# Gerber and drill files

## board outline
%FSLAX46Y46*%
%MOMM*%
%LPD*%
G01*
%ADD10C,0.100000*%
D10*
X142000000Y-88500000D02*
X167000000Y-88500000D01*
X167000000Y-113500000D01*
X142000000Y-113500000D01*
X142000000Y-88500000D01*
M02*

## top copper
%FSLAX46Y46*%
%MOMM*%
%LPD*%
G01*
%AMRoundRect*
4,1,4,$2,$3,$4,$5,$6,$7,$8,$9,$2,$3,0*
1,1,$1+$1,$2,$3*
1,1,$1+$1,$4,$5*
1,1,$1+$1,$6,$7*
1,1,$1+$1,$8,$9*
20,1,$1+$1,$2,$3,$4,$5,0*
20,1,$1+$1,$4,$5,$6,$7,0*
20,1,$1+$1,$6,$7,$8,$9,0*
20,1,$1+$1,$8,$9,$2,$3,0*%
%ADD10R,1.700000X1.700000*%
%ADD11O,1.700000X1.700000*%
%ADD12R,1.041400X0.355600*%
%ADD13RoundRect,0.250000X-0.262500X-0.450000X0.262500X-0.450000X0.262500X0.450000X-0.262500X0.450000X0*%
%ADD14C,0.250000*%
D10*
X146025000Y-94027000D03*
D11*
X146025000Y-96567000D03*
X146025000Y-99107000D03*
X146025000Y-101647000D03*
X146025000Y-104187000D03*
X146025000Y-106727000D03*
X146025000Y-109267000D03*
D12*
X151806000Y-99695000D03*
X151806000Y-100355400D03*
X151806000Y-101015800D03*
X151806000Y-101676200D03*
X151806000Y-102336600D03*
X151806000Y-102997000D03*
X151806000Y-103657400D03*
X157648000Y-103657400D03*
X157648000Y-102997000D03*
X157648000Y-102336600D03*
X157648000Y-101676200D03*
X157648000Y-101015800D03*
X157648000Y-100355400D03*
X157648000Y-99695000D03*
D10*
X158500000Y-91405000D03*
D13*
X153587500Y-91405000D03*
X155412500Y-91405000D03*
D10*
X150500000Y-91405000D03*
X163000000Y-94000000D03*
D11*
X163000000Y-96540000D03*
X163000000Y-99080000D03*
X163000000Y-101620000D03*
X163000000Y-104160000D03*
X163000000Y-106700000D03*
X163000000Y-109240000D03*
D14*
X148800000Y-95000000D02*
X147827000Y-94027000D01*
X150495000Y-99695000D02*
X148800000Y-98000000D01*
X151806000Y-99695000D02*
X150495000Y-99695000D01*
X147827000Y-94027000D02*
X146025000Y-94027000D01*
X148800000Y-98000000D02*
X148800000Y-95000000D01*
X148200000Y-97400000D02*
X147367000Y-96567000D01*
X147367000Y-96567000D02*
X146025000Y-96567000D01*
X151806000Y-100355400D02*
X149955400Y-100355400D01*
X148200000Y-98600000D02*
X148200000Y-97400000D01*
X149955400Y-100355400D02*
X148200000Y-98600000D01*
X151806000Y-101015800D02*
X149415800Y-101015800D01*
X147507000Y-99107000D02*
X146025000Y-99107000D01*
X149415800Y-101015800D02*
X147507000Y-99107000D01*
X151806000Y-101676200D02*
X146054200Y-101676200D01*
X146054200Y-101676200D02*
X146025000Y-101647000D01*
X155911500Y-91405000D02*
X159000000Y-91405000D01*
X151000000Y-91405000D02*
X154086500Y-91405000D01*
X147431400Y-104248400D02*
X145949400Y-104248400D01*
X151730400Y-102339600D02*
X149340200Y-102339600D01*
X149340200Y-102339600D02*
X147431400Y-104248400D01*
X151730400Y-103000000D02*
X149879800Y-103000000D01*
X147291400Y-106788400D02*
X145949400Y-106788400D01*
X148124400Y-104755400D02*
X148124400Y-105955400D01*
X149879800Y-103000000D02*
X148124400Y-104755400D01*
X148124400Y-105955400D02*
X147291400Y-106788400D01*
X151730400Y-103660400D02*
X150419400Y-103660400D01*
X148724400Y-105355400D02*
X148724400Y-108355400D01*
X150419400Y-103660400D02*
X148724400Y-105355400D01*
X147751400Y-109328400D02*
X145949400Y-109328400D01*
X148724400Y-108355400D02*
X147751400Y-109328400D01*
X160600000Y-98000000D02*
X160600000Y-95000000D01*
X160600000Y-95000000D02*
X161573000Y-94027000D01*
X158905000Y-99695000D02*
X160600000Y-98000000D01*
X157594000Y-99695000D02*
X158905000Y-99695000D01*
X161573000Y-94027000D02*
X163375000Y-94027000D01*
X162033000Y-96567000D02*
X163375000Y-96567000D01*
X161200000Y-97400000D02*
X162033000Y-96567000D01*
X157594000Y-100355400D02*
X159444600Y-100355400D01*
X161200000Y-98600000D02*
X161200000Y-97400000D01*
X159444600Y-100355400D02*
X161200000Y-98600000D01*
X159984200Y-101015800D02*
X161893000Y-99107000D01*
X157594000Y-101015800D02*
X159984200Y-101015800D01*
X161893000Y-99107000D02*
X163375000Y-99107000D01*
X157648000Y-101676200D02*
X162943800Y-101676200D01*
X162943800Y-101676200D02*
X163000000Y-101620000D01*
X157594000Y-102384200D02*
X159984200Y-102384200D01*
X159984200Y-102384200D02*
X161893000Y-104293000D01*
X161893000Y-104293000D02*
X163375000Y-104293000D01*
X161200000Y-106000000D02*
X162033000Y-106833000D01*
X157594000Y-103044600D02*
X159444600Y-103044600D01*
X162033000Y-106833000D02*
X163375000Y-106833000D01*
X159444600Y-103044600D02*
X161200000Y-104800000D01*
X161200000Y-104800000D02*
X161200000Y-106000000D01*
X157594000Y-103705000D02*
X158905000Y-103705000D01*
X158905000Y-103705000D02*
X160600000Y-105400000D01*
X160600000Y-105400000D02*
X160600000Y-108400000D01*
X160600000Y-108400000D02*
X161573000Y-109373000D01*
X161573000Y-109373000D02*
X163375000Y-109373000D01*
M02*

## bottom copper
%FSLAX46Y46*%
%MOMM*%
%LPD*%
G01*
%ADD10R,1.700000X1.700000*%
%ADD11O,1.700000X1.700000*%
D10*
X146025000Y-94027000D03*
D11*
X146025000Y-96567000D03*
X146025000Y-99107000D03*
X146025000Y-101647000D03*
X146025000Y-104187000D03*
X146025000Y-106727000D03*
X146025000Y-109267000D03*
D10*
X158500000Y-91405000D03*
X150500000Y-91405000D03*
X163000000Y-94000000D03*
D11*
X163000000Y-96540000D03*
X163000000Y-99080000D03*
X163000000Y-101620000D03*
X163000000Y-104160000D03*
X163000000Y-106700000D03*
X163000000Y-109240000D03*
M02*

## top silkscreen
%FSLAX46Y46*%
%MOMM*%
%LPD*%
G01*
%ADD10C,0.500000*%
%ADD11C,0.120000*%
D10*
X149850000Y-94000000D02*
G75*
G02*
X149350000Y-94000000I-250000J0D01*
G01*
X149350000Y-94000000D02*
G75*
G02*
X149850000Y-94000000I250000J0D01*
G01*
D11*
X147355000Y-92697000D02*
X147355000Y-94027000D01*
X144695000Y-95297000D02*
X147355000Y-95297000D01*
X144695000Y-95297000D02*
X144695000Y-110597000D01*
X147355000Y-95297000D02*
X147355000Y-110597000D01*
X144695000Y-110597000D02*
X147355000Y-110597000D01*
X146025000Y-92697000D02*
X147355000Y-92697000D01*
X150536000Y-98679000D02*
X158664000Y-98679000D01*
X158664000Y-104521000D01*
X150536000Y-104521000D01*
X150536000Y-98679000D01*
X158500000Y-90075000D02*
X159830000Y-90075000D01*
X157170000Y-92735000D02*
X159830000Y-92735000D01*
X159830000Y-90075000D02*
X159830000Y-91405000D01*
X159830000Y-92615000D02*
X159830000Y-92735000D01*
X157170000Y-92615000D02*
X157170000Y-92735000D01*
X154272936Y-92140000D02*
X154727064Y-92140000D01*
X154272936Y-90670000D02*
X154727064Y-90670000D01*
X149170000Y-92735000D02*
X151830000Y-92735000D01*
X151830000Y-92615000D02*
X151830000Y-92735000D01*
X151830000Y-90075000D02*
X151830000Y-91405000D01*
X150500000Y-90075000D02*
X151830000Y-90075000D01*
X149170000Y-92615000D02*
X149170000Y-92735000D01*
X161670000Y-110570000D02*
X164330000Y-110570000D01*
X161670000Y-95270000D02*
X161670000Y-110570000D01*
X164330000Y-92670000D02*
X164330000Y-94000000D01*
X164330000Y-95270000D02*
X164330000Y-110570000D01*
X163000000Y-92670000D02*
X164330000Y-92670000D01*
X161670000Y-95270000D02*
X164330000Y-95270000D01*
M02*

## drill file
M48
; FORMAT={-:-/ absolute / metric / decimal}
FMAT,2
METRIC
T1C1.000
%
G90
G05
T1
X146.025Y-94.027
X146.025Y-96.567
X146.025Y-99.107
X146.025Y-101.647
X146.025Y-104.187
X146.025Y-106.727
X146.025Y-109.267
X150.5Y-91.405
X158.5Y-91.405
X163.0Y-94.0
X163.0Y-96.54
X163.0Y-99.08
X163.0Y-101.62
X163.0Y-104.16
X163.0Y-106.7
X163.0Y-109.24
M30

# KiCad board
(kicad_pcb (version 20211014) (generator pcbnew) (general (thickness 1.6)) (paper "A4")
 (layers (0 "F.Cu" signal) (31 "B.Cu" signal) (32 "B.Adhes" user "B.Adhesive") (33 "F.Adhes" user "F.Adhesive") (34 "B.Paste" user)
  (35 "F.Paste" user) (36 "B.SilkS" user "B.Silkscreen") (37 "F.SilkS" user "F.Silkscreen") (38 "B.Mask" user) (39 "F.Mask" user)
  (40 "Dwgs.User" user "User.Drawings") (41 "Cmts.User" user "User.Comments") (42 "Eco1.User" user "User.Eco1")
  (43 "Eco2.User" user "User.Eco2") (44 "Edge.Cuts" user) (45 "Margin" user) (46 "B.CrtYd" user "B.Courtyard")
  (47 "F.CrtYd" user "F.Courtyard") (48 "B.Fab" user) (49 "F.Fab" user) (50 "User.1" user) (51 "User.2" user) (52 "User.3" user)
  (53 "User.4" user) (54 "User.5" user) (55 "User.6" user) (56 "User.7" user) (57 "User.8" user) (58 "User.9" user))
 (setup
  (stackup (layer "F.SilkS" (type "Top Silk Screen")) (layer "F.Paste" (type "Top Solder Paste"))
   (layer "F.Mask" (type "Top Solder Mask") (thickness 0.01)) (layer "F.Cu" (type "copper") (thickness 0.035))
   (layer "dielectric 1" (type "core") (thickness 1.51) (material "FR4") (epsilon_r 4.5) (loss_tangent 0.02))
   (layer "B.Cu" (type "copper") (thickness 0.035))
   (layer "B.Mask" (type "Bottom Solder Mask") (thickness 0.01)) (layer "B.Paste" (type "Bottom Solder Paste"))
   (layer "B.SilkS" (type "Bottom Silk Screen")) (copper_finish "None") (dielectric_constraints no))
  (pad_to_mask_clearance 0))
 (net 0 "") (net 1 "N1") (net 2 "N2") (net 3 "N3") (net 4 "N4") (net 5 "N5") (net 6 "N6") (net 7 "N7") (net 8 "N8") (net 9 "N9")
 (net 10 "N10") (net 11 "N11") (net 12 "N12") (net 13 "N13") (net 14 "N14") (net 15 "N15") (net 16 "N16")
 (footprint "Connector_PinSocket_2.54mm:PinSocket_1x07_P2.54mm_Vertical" (layer "F.Cu") (at 146.025 94.027)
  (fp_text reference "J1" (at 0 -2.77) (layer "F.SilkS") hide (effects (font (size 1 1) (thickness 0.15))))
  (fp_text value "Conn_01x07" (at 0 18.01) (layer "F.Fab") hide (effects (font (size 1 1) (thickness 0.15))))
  (fp_line (start 1.33 -1.33) (end 1.33 0) (layer "F.SilkS") (width 0.12))
  (fp_line (start -1.33 1.27) (end 1.33 1.27) (layer "F.SilkS") (width 0.12))
  (fp_line (start -1.33 1.27) (end -1.33 16.57) (layer "F.SilkS") (width 0.12))
  (fp_line (start 1.33 1.27) (end 1.33 16.57) (layer "F.SilkS") (width 0.12))
  (fp_line (start -1.33 16.57) (end 1.33 16.57) (layer "F.SilkS") (width 0.12))
  (fp_line (start 0 -1.33) (end 1.33 -1.33) (layer "F.SilkS") (width 0.12))
  (pad "1" thru_hole rect (at 0 0) (size 1.7 1.7) (drill 1) (layers *.Cu *.Mask) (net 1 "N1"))
  (pad "2" thru_hole oval (at 0 2.54) (size 1.7 1.7) (drill 1) (layers *.Cu *.Mask) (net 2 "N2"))
  (pad "3" thru_hole oval (at 0 5.08) (size 1.7 1.7) (drill 1) (layers *.Cu *.Mask) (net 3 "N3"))
  (pad "4" thru_hole oval (at 0 7.62) (size 1.7 1.7) (drill 1) (layers *.Cu *.Mask) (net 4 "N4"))
  (pad "5" thru_hole oval (at 0 10.16) (size 1.7 1.7) (drill 1) (layers *.Cu *.Mask) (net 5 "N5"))
  (pad "6" thru_hole oval (at 0 12.7) (size 1.7 1.7) (drill 1) (layers *.Cu *.Mask) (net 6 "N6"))
  (pad "7" thru_hole oval (at 0 15.24) (size 1.7 1.7) (drill 1) (layers *.Cu *.Mask) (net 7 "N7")))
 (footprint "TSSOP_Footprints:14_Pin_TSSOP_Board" (layer "F.Cu") (at 154.727 103.759)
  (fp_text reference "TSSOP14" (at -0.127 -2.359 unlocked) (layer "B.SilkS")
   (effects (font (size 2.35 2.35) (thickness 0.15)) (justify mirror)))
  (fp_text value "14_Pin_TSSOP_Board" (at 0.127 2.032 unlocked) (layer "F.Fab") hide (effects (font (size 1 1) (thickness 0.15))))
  (fp_rect (start -4.191 -5.08) (end 3.937 0.762) (layer "F.SilkS") (width 0.12) (fill none))
  (pad "1" smd rect (at -2.921 -4.064) (size 1.0414 0.3556) (layers "F.Cu" "F.Paste" "F.Mask") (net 1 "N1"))
  (pad "2" smd rect (at -2.921 -3.4036) (size 1.0414 0.3556) (layers "F.Cu" "F.Paste" "F.Mask") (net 2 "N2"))
  (pad "3" smd rect (at -2.921 -2.7432) (size 1.0414 0.3556) (layers "F.Cu" "F.Paste" "F.Mask") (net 3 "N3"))
  (pad "4" smd rect (at -2.921 -2.0828) (size 1.0414 0.3556) (layers "F.Cu" "F.Paste" "F.Mask") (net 4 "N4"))
  (pad "5" smd rect (at -2.921 -1.4224) (size 1.0414 0.3556) (layers "F.Cu" "F.Paste" "F.Mask") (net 5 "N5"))
  (pad "6" smd rect (at -2.921 -0.762) (size 1.0414 0.3556) (layers "F.Cu" "F.Paste" "F.Mask") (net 6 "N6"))
  (pad "7" smd rect (at -2.921 -0.1016) (size 1.0414 0.3556) (layers "F.Cu" "F.Paste" "F.Mask") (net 7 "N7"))
  (pad "8" smd rect (at 2.921 -0.1016) (size 1.0414 0.3556) (layers "F.Cu" "F.Paste" "F.Mask") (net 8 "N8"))
  (pad "9" smd rect (at 2.921 -0.762) (size 1.0414 0.3556) (layers "F.Cu" "F.Paste" "F.Mask") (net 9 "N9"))
  (pad "10" smd rect (at 2.921 -1.4224) (size 1.0414 0.3556) (layers "F.Cu" "F.Paste" "F.Mask") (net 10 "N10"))
  (pad "11" smd rect (at 2.921 -2.0828) (size 1.0414 0.3556) (layers "F.Cu" "F.Paste" "F.Mask") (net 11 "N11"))
  (pad "12" smd rect (at 2.921 -2.7432) (size 1.0414 0.3556) (layers "F.Cu" "F.Paste" "F.Mask") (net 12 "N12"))
  (pad "13" smd rect (at 2.921 -3.4036) (size 1.0414 0.3556) (layers "F.Cu" "F.Paste" "F.Mask") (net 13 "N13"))
  (pad "14" smd rect (at 2.921 -4.064) (size 1.0414 0.3556) (layers "F.Cu" "F.Paste" "F.Mask") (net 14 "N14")))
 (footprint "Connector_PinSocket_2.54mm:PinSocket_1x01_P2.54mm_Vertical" (layer "F.Cu") (at 158.5 91.405)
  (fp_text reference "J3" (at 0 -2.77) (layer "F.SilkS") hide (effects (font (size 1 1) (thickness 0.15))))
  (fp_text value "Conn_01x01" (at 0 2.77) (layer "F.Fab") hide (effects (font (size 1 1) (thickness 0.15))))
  (fp_line (start 0 -1.33) (end 1.33 -1.33) (layer "F.SilkS") (width 0.12))
  (fp_line (start -1.33 1.33) (end 1.33 1.33) (layer "F.SilkS") (width 0.12))
  (fp_line (start 1.33 -1.33) (end 1.33 0) (layer "F.SilkS") (width 0.12))
  (fp_line (start 1.33 1.21) (end 1.33 1.33) (layer "F.SilkS") (width 0.12))
  (fp_line (start -1.33 1.21) (end -1.33 1.33) (layer "F.SilkS") (width 0.12))
  (pad "1" thru_hole rect (at 0 0) (size 1.7 1.7) (drill 1) (layers *.Cu *.Mask) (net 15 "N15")))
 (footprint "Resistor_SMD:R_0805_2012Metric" (layer "F.Cu") (at 154.5 91.405)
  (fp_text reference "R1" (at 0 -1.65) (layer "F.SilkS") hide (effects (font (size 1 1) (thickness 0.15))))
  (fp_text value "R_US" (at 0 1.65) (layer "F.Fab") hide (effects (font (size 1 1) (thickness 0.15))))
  (fp_line (start -0.227064 0.735) (end 0.227064 0.735) (layer "F.SilkS") (width 0.12))
  (fp_line (start -0.227064 -0.735) (end 0.227064 -0.735) (layer "F.SilkS") (width 0.12))
  (pad "1" smd roundrect (at -0.9125 0) (size 1.025 1.4) (layers "F.Cu" "F.Paste" "F.Mask") (roundrect_rratio 0.243902) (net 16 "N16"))
  (pad "2" smd roundrect (at 0.9125 0) (size 1.025 1.4) (layers "F.Cu" "F.Paste" "F.Mask") (roundrect_rratio 0.243902) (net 15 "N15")))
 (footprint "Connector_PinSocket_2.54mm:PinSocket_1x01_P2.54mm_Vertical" (layer "F.Cu") (at 150.5 91.405)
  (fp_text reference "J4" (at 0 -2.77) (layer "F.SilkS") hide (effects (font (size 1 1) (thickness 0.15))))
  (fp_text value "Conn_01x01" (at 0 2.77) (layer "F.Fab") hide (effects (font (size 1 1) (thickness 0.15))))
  (fp_line (start -1.33 1.33) (end 1.33 1.33) (layer "F.SilkS") (width 0.12))
  (fp_line (start 1.33 1.21) (end 1.33 1.33) (layer "F.SilkS") (width 0.12))
  (fp_line (start 1.33 -1.33) (end 1.33 0) (layer "F.SilkS") (width 0.12))
  (fp_line (start 0 -1.33) (end 1.33 -1.33) (layer "F.SilkS") (width 0.12))
  (fp_line (start -1.33 1.21) (end -1.33 1.33) (layer "F.SilkS") (width 0.12))
  (pad "1" thru_hole rect (at 0 0) (size 1.7 1.7) (drill 1) (layers *.Cu *.Mask) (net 16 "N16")))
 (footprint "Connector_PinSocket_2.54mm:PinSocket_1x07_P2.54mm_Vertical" (layer "F.Cu") (at 163 94)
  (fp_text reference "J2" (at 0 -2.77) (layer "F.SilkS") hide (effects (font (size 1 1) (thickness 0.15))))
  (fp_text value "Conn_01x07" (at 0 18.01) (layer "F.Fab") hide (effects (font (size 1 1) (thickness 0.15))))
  (fp_line (start -1.33 16.57) (end 1.33 16.57) (layer "F.SilkS") (width 0.12))
  (fp_line (start -1.33 1.27) (end -1.33 16.57) (layer "F.SilkS") (width 0.12))
  (fp_line (start 1.33 -1.33) (end 1.33 0) (layer "F.SilkS") (width 0.12))
  (fp_line (start 1.33 1.27) (end 1.33 16.57) (layer "F.SilkS") (width 0.12))
  (fp_line (start 0 -1.33) (end 1.33 -1.33) (layer "F.SilkS") (width 0.12))
  (fp_line (start -1.33 1.27) (end 1.33 1.27) (layer "F.SilkS") (width 0.12))
  (pad "1" thru_hole rect (at 0 0) (size 1.7 1.7) (drill 1) (layers *.Cu *.Mask) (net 14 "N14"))
  (pad "2" thru_hole oval (at 0 2.54) (size 1.7 1.7) (drill 1) (layers *.Cu *.Mask) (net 13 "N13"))
  (pad "3" thru_hole oval (at 0 5.08) (size 1.7 1.7) (drill 1) (layers *.Cu *.Mask) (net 12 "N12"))
  (pad "4" thru_hole oval (at 0 7.62) (size 1.7 1.7) (drill 1) (layers *.Cu *.Mask) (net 11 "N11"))
  (pad "5" thru_hole oval (at 0 10.16) (size 1.7 1.7) (drill 1) (layers *.Cu *.Mask) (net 10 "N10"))
  (pad "6" thru_hole oval (at 0 12.7) (size 1.7 1.7) (drill 1) (layers *.Cu *.Mask) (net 9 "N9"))
  (pad "7" thru_hole oval (at 0 15.24) (size 1.7 1.7) (drill 1) (layers *.Cu *.Mask) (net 8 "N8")))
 (gr_circle (center 149.6 94) (end 150 94) (layer "F.SilkS") (width 0.2) (fill solid))
 (gr_rect (start 142 88.5) (end 167 113.5) (layer "Edge.Cuts") (width 0.1) (fill none))
 (segment (start 148.8 95) (end 147.827 94.027) (width 0.25) (layer "F.Cu") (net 1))
 (segment (start 150.495 99.695) (end 148.8 98) (width 0.25) (layer "F.Cu") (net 1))
 (segment (start 151.806 99.695) (end 150.495 99.695) (width 0.25) (layer "F.Cu") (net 1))
 (segment (start 147.827 94.027) (end 146.025 94.027) (width 0.25) (layer "F.Cu") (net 1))
 (segment (start 148.8 98) (end 148.8 95) (width 0.25) (layer "F.Cu") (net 1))
 (segment (start 148.2 97.4) (end 147.367 96.567) (width 0.25) (layer "F.Cu") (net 2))
 (segment (start 147.367 96.567) (end 146.025 96.567) (width 0.25) (layer "F.Cu") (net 2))
 (segment (start 151.806 100.3554) (end 149.9554 100.3554) (width 0.25) (layer "F.Cu") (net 2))
 (segment (start 148.2 98.6) (end 148.2 97.4) (width 0.25) (layer "F.Cu") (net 2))
 (segment (start 149.9554 100.3554) (end 148.2 98.6) (width 0.25) (layer "F.Cu") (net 2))
 (segment (start 151.806 101.0158) (end 149.4158 101.0158) (width 0.25) (layer "F.Cu") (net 3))
 (segment (start 147.507 99.107) (end 146.025 99.107) (width 0.25) (layer "F.Cu") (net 3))
 (segment (start 149.4158 101.0158) (end 147.507 99.107) (width 0.25) (layer "F.Cu") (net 3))
 (segment (start 151.806 101.6762) (end 146.0542 101.6762) (width 0.25) (layer "F.Cu") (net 4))
 (segment (start 146.0542 101.6762) (end 146.025 101.647) (width 0.25) (layer "F.Cu") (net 4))
 (segment (start 155.9115 91.405) (end 159 91.405) (width 0.25) (layer "F.Cu") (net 15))
 (segment (start 151 91.405) (end 154.0865 91.405) (width 0.25) (layer "F.Cu") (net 16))
 (segment (start 147.4314 104.2484) (end 145.9494 104.2484) (width 0.25) (layer "F.Cu") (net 5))
 (segment (start 151.7304 102.3396) (end 149.3402 102.3396) (width 0.25) (layer "F.Cu") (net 5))
 (segment (start 149.3402 102.3396) (end 147.4314 104.2484) (width 0.25) (layer "F.Cu") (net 5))
 (segment (start 151.7304 103) (end 149.8798 103) (width 0.25) (layer "F.Cu") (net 6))
 (segment (start 147.2914 106.7884) (end 145.9494 106.7884) (width 0.25) (layer "F.Cu") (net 6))
 (segment (start 148.1244 104.7554) (end 148.1244 105.9554) (width 0.25) (layer "F.Cu") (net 6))
 (segment (start 149.8798 103) (end 148.1244 104.7554) (width 0.25) (layer "F.Cu") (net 6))
 (segment (start 148.1244 105.9554) (end 147.2914 106.7884) (width 0.25) (layer "F.Cu") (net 6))
 (segment (start 151.7304 103.6604) (end 150.4194 103.6604) (width 0.25) (layer "F.Cu") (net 7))
 (segment (start 148.7244 105.3554) (end 148.7244 108.3554) (width 0.25) (layer "F.Cu") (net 7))
 (segment (start 150.4194 103.6604) (end 148.7244 105.3554) (width 0.25) (layer "F.Cu") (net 7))
 (segment (start 147.7514 109.3284) (end 145.9494 109.3284) (width 0.25) (layer "F.Cu") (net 7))
 (segment (start 148.7244 108.3554) (end 147.7514 109.3284) (width 0.25) (layer "F.Cu") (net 7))
 (segment (start 160.6 98) (end 160.6 95) (width 0.25) (layer "F.Cu") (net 14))
 (segment (start 160.6 95) (end 161.573 94.027) (width 0.25) (layer "F.Cu") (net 14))
 (segment (start 158.905 99.695) (end 160.6 98) (width 0.25) (layer "F.Cu") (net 14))
 (segment (start 157.594 99.695) (end 158.905 99.695) (width 0.25) (layer "F.Cu") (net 14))
 (segment (start 161.573 94.027) (end 163.375 94.027) (width 0.25) (layer "F.Cu") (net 14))
 (segment (start 162.033 96.567) (end 163.375 96.567) (width 0.25) (layer "F.Cu") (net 13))
 (segment (start 161.2 97.4) (end 162.033 96.567) (width 0.25) (layer "F.Cu") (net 13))
 (segment (start 157.594 100.3554) (end 159.4446 100.3554) (width 0.25) (layer "F.Cu") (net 13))
 (segment (start 161.2 98.6) (end 161.2 97.4) (width 0.25) (layer "F.Cu") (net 13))
 (segment (start 159.4446 100.3554) (end 161.2 98.6) (width 0.25) (layer "F.Cu") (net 13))
 (segment (start 159.9842 101.0158) (end 161.893 99.107) (width 0.25) (layer "F.Cu") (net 12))
 (segment (start 157.594 101.0158) (end 159.9842 101.0158) (width 0.25) (layer "F.Cu") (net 12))
 (segment (start 161.893 99.107) (end 163.375 99.107) (width 0.25) (layer "F.Cu") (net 12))
 (segment (start 157.648 101.6762) (end 162.9438 101.6762) (width 0.25) (layer "F.Cu") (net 11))
 (segment (start 162.9438 101.6762) (end 163 101.62) (width 0.25) (layer "F.Cu") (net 11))
 (segment (start 157.594 102.3842) (end 159.9842 102.3842) (width 0.25) (layer "F.Cu") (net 10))
 (segment (start 159.9842 102.3842) (end 161.893 104.293) (width 0.25) (layer "F.Cu") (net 10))
 (segment (start 161.893 104.293) (end 163.375 104.293) (width 0.25) (layer "F.Cu") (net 10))
 (segment (start 161.2 106) (end 162.033 106.833) (width 0.25) (layer "F.Cu") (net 9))
 (segment (start 157.594 103.0446) (end 159.4446 103.0446) (width 0.25) (layer "F.Cu") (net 9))
 (segment (start 162.033 106.833) (end 163.375 106.833) (width 0.25) (layer "F.Cu") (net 9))
 (segment (start 159.4446 103.0446) (end 161.2 104.8) (width 0.25) (layer "F.Cu") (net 9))
 (segment (start 161.2 104.8) (end 161.2 106) (width 0.25) (layer "F.Cu") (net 9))
 (segment (start 157.594 103.705) (end 158.905 103.705) (width 0.25) (layer "F.Cu") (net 8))
 (segment (start 158.905 103.705) (end 160.6 105.4) (width 0.25) (layer "F.Cu") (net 8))
 (segment (start 160.6 105.4) (end 160.6 108.4) (width 0.25) (layer "F.Cu") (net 8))
 (segment (start 160.6 108.4) (end 161.573 109.373) (width 0.25) (layer "F.Cu") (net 8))
 (segment (start 161.573 109.373) (end 163.375 109.373) (width 0.25) (layer "F.Cu") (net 8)))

